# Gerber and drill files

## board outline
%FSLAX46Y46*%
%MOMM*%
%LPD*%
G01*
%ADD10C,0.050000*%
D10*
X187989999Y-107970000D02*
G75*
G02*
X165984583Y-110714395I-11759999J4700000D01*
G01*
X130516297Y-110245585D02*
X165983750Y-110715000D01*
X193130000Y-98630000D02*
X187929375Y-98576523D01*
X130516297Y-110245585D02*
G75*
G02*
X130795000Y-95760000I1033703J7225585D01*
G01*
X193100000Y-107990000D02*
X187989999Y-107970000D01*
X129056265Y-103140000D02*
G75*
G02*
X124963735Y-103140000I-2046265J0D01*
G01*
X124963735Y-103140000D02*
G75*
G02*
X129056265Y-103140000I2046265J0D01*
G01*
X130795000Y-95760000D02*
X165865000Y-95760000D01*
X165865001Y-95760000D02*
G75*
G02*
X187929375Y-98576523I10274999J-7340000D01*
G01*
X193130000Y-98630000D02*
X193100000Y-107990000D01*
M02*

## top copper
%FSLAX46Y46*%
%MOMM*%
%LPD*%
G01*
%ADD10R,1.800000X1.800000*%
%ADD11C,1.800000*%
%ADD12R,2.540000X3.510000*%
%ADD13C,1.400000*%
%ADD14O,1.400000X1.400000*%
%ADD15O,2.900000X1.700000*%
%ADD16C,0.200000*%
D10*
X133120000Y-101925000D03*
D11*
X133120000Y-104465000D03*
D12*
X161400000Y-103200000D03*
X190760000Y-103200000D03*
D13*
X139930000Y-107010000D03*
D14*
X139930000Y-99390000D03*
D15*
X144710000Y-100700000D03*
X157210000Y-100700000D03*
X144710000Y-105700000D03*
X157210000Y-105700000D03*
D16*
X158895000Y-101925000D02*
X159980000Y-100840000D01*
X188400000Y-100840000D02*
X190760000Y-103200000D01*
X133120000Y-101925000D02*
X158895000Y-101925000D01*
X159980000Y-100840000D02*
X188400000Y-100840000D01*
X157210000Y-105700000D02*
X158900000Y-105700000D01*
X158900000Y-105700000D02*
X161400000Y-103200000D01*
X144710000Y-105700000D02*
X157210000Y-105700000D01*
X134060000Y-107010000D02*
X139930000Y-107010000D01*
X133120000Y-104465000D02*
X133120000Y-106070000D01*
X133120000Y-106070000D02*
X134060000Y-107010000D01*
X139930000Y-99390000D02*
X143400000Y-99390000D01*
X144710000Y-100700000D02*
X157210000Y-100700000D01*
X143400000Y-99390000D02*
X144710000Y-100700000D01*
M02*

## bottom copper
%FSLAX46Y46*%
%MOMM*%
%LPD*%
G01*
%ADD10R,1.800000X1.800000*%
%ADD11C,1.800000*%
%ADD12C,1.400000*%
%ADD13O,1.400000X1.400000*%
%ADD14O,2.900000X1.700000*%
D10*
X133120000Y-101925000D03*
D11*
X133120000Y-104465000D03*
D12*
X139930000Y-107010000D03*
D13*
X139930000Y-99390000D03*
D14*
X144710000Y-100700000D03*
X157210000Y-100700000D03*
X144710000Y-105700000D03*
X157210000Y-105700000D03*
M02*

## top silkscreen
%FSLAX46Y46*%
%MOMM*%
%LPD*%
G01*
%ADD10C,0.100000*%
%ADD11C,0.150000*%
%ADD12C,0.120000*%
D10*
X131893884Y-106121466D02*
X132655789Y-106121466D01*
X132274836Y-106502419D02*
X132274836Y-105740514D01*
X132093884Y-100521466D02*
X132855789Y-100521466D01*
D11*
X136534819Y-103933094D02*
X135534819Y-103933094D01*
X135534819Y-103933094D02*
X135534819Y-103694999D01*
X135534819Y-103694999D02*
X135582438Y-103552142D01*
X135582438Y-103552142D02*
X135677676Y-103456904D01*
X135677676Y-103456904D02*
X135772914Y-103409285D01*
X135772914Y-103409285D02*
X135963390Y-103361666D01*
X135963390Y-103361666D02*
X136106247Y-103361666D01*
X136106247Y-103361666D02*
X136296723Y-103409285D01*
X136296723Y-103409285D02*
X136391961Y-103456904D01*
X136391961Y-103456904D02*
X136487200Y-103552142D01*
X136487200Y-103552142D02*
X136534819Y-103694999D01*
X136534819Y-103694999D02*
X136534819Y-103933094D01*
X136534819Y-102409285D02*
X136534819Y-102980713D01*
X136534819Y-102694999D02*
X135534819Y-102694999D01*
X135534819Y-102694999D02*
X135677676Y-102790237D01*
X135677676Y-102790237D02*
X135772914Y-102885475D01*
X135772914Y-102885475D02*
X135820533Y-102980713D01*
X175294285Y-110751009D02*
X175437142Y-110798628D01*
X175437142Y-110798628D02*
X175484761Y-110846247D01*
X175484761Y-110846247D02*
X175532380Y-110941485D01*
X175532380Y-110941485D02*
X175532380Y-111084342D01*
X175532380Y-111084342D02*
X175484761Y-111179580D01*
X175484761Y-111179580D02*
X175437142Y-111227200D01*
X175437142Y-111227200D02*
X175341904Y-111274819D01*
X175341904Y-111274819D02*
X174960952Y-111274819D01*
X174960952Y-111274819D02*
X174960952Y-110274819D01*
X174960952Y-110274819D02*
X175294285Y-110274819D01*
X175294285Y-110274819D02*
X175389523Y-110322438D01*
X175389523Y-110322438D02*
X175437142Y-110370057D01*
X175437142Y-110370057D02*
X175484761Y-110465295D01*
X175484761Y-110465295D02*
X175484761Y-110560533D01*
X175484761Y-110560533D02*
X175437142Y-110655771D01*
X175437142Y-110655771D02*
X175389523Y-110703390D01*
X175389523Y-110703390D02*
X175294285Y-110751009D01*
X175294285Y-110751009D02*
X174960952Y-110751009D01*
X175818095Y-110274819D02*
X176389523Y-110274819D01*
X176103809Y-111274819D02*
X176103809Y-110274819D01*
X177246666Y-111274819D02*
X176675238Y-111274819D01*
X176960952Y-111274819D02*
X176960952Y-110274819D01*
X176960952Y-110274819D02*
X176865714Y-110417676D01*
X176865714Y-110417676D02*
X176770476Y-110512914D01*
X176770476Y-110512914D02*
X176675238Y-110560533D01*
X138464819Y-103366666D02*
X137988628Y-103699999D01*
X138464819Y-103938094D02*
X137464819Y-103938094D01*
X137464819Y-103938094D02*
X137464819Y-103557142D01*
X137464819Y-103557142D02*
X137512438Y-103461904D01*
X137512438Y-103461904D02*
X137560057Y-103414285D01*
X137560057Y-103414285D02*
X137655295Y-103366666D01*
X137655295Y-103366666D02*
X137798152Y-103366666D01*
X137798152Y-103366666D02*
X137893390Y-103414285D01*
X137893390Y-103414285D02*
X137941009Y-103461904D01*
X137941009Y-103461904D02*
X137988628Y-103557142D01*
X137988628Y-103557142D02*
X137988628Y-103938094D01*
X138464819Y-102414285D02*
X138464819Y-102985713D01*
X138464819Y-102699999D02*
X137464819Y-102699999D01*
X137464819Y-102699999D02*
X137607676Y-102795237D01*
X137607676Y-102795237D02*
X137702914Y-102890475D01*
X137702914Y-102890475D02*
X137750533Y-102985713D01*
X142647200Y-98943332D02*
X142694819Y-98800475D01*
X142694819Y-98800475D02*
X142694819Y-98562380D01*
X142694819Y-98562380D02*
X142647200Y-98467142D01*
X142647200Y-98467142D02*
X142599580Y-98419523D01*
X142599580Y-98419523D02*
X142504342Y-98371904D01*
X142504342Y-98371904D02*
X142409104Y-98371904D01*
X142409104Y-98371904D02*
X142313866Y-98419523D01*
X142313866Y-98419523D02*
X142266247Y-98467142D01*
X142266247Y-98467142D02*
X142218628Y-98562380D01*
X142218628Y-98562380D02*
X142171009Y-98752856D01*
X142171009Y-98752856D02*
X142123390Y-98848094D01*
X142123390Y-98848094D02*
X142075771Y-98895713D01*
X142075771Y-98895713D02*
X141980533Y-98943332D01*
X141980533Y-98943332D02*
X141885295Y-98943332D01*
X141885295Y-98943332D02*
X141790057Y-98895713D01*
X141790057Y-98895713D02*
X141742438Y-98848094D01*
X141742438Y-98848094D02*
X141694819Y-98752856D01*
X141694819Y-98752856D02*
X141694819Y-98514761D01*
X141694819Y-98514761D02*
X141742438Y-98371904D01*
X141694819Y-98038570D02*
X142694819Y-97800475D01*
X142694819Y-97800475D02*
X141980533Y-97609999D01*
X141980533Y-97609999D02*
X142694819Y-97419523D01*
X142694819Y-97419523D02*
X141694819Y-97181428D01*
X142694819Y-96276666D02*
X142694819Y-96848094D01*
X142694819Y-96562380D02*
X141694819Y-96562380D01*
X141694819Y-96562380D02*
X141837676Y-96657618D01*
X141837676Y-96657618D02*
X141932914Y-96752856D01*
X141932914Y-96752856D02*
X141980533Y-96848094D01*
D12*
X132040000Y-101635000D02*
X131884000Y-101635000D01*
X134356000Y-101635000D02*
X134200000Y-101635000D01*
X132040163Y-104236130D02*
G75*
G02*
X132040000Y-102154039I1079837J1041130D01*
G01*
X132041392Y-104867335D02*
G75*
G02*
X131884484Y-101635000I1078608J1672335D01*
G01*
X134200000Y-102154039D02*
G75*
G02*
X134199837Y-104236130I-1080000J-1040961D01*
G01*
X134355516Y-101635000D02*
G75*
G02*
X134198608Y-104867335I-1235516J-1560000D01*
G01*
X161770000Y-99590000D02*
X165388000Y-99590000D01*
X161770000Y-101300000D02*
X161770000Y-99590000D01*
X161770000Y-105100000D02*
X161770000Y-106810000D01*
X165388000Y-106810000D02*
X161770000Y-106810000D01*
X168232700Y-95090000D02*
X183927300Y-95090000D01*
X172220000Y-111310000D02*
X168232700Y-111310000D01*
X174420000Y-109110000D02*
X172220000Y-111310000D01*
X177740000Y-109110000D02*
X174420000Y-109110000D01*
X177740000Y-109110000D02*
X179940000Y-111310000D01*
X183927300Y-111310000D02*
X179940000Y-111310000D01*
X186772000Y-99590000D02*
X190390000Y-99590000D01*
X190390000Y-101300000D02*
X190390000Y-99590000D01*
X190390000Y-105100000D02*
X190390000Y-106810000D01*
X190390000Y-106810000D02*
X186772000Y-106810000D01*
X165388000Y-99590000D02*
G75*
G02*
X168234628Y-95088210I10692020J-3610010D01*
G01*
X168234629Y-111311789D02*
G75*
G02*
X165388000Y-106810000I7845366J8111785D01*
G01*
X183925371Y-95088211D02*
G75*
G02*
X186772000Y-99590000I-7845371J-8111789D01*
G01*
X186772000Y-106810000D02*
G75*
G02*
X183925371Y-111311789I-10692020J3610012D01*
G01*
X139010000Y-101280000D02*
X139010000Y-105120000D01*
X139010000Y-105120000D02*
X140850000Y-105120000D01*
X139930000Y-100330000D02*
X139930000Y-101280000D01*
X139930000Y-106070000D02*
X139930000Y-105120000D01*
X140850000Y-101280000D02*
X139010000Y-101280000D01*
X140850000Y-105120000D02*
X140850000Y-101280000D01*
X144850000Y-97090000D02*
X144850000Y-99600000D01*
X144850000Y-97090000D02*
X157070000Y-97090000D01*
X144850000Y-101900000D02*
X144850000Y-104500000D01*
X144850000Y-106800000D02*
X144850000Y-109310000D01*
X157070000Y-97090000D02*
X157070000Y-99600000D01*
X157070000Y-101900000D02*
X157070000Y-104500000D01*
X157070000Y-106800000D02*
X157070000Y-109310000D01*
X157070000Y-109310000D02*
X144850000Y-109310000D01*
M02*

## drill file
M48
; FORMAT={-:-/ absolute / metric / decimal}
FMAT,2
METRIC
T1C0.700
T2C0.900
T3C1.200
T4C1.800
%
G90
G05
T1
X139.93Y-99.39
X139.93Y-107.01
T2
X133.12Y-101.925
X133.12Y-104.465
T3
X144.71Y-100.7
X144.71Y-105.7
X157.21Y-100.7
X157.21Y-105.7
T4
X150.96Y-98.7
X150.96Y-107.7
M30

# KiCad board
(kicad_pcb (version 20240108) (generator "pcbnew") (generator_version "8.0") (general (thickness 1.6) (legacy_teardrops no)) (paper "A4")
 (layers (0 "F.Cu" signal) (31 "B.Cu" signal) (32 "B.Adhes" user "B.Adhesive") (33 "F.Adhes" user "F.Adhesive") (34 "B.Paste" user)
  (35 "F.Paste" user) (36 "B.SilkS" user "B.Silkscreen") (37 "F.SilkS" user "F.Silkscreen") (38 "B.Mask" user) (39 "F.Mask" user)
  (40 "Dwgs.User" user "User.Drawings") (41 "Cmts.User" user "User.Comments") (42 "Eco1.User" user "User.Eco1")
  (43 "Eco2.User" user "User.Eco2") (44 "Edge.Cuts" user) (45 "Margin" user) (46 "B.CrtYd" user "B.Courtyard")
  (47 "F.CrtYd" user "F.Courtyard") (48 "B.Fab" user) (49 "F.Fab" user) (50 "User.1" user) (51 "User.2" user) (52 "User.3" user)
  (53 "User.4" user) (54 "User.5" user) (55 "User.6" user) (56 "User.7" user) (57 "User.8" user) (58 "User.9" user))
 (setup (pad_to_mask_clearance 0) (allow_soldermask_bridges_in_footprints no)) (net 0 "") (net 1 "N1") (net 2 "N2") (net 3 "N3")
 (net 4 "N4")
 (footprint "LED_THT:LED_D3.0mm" (layer "F.Cu") (at 133.12 101.925 -90)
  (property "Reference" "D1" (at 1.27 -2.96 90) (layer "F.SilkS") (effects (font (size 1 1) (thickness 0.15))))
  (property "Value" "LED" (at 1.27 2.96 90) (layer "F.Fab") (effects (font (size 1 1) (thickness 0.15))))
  (fp_line (start -0.29 1.08) (end -0.29 1.236) (stroke (width 0.12) (type solid)) (layer "F.SilkS"))
  (fp_line (start -0.29 -1.236) (end -0.29 -1.08) (stroke (width 0.12) (type solid)) (layer "F.SilkS"))
  (fp_arc (start 2.31113 1.079837) (mid 1.270117 1.5) (end 0.229039 1.08) (stroke (width 0.12) (type solid)) (layer "F.SilkS"))
  (fp_arc (start 2.942335 1.078608) (mid 1.366487 1.987659) (end -0.29 1.235516) (stroke (width 0.12) (type solid)) (layer "F.SilkS"))
  (fp_arc (start 0.229039 -1.08) (mid 1.270117 -1.5) (end 2.31113 -1.079837) (stroke (width 0.12) (type solid)) (layer "F.SilkS"))
  (fp_arc (start -0.29 -1.235516) (mid 1.366487 -1.987659) (end 2.942335 -1.078608) (stroke (width 0.12) (type solid)) (layer "F.SilkS"))
  (pad "1" thru_hole rect (at 0 0 270) (size 1.8 1.8) (drill 0.9) (layers "*.Cu" "*.Mask") (remove_unused_layers no) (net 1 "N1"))
  (pad "2" thru_hole circle (at 2.54 0 270) (size 1.8 1.8) (drill 0.9) (layers "*.Cu" "*.Mask") (remove_unused_layers no) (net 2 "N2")))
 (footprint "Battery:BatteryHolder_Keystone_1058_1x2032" (layer "F.Cu") (at 176.08 103.2)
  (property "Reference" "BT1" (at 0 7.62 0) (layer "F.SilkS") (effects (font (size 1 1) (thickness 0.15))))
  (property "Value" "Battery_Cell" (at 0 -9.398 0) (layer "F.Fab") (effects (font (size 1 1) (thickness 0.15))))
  (fp_line (start -14.31 -3.61) (end -10.692 -3.61) (stroke (width 0.12) (type solid)) (layer "F.SilkS"))
  (fp_line (start -14.31 -1.9) (end -14.31 -3.61) (stroke (width 0.12) (type solid)) (layer "F.SilkS"))
  (fp_line (start -14.31 1.9) (end -14.31 3.61) (stroke (width 0.12) (type solid)) (layer "F.SilkS"))
  (fp_line (start -10.692 3.61) (end -14.31 3.61) (stroke (width 0.12) (type solid)) (layer "F.SilkS"))
  (fp_line (start -7.8473 -8.11) (end 7.8473 -8.11) (stroke (width 0.12) (type solid)) (layer "F.SilkS"))
  (fp_line (start -3.86 8.11) (end -7.8473 8.11) (stroke (width 0.12) (type solid)) (layer "F.SilkS"))
  (fp_line (start -1.66 5.91) (end -3.86 8.11) (stroke (width 0.12) (type solid)) (layer "F.SilkS"))
  (fp_line (start 1.66 5.91) (end -1.66 5.91) (stroke (width 0.12) (type solid)) (layer "F.SilkS"))
  (fp_line (start 1.66 5.91) (end 3.86 8.11) (stroke (width 0.12) (type solid)) (layer "F.SilkS"))
  (fp_line (start 7.8473 8.11) (end 3.86 8.11) (stroke (width 0.12) (type solid)) (layer "F.SilkS"))
  (fp_line (start 10.692 -3.61) (end 14.31 -3.61) (stroke (width 0.12) (type solid)) (layer "F.SilkS"))
  (fp_line (start 14.31 -1.9) (end 14.31 -3.61) (stroke (width 0.12) (type solid)) (layer "F.SilkS"))
  (fp_line (start 14.31 1.9) (end 14.31 3.61) (stroke (width 0.12) (type solid)) (layer "F.SilkS"))
  (fp_line (start 14.31 3.61) (end 10.692 3.61) (stroke (width 0.12) (type solid)) (layer "F.SilkS"))
  (fp_arc (start -10.692 -3.61) (mid -9.538084 -6.031244) (end -7.845371 -8.111789) (stroke (width 0.12) (type solid)) (layer "F.SilkS"))
  (fp_arc (start -7.845371 8.111789) (mid -9.538085 6.031244) (end -10.692 3.61) (stroke (width 0.12) (type solid)) (layer "F.SilkS"))
  (fp_arc (start 7.845371 -8.111789) (mid 9.538085 -6.031244) (end 10.692 -3.61) (stroke (width 0.12) (type solid)) (layer "F.SilkS"))
  (fp_arc (start 10.692 3.61) (mid 9.538084 6.031244) (end 7.845371 8.111789) (stroke (width 0.12) (type solid)) (layer "F.SilkS"))
  (pad "1" smd rect (at -14.68 0) (size 2.54 3.51) (layers "F.Cu" "F.Paste" "F.Mask") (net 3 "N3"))
  (pad "2" smd rect (at 14.68 0) (size 2.54 3.51) (layers "F.Cu" "F.Paste" "F.Mask") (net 1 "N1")))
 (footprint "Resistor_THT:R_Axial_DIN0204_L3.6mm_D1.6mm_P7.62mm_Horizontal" (layer "F.Cu") (at 139.93 107.01 90)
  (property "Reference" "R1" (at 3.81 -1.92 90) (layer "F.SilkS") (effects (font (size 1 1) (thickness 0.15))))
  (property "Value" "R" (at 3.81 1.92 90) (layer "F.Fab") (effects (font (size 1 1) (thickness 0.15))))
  (fp_line (start 5.73 -0.92) (end 1.89 -0.92) (stroke (width 0.12) (type solid)) (layer "F.SilkS"))
  (fp_line (start 1.89 -0.92) (end 1.89 0.92) (stroke (width 0.12) (type solid)) (layer "F.SilkS"))
  (fp_line (start 6.68 0) (end 5.73 0) (stroke (width 0.12) (type solid)) (layer "F.SilkS"))
  (fp_line (start 0.94 0) (end 1.89 0) (stroke (width 0.12) (type solid)) (layer "F.SilkS"))
  (fp_line (start 5.73 0.92) (end 5.73 -0.92) (stroke (width 0.12) (type solid)) (layer "F.SilkS"))
  (fp_line (start 1.89 0.92) (end 5.73 0.92) (stroke (width 0.12) (type solid)) (layer "F.SilkS"))
  (pad "1" thru_hole circle (at 0 0 90) (size 1.4 1.4) (drill 0.7) (layers "*.Cu" "*.Mask") (remove_unused_layers no) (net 2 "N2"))
  (pad "2" thru_hole oval (at 7.62 0 90) (size 1.4 1.4) (drill 0.7) (layers "*.Cu" "*.Mask") (remove_unused_layers no) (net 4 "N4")))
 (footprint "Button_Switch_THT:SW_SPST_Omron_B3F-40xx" (layer "F.Cu") (at 144.71 100.7)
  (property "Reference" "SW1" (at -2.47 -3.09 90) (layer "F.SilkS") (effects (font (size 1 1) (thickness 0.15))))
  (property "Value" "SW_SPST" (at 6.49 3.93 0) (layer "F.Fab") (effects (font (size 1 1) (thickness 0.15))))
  (fp_line (start 0.14 -3.61) (end 0.14 -1.1) (stroke (width 0.12) (type default)) (layer "F.SilkS"))
  (fp_line (start 0.14 -3.61) (end 12.36 -3.61) (stroke (width 0.12) (type default)) (layer "F.SilkS"))
  (fp_line (start 0.14 1.2) (end 0.14 3.8) (stroke (width 0.12) (type default)) (layer "F.SilkS"))
  (fp_line (start 0.14 6.1) (end 0.14 8.61) (stroke (width 0.12) (type default)) (layer "F.SilkS"))
  (fp_line (start 12.36 -3.61) (end 12.36 -1.1) (stroke (width 0.12) (type default)) (layer "F.SilkS"))
  (fp_line (start 12.36 1.2) (end 12.36 3.8) (stroke (width 0.12) (type default)) (layer "F.SilkS"))
  (fp_line (start 12.36 6.1) (end 12.36 8.61) (stroke (width 0.12) (type default)) (layer "F.SilkS"))
  (fp_line (start 12.36 8.61) (end 0.14 8.61) (stroke (width 0.12) (type default)) (layer "F.SilkS"))
  (pad "" np_thru_hole circle (at 6.25 -2) (size 1.8 1.8) (drill 1.8) (layers "F&B.Cu" "*.Mask"))
  (pad "" np_thru_hole circle (at 6.25 7) (size 1.8 1.8) (drill 1.8) (layers "F&B.Cu" "*.Mask"))
  (pad "1" thru_hole oval (at 0 0) (size 2.9 1.7) (drill 1.2) (layers "*.Cu" "*.Mask") (remove_unused_layers no) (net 4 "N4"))
  (pad "1" thru_hole oval (at 12.5 0) (size 2.9 1.7) (drill 1.2) (layers "*.Cu" "*.Mask") (remove_unused_layers no) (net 4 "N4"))
  (pad "2" thru_hole oval (at 0 5) (size 2.9 1.7) (drill 1.2) (layers "*.Cu" "*.Mask") (remove_unused_layers no) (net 3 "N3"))
  (pad "2" thru_hole oval (at 12.5 5) (size 2.9 1.7) (drill 1.2) (layers "*.Cu" "*.Mask") (remove_unused_layers no) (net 3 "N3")))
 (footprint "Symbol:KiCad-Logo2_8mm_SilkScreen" (layer "B.Cu") (at 173.409893 102.476424 180)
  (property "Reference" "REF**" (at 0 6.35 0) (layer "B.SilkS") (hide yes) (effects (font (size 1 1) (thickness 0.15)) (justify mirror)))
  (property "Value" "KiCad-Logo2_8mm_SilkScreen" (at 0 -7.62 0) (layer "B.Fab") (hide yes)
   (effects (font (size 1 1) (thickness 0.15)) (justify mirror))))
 (gr_arc (start 187.989999 107.97) (mid 177.797296 115.837067) (end 165.984583 110.714395) (stroke (width 0.05) (type default))
  (layer "Edge.Cuts"))
 (gr_line (start 130.516297 110.245585) (end 165.98375 110.715) (stroke (width 0.05) (type default)) (layer "Edge.Cuts"))
 (gr_line (start 193.13 98.63) (end 187.929375 98.576523) (stroke (width 0.05) (type default)) (layer "Edge.Cuts"))
 (gr_arc (start 130.516297 110.245585) (mid 124.252199 102.87959) (end 130.795 95.76) (stroke (width 0.05) (type default))
  (layer "Edge.Cuts"))
 (gr_line (start 193.1 107.99) (end 187.989999 107.97) (stroke (width 0.05) (type default)) (layer "Edge.Cuts"))
 (gr_circle (center 127.01 103.14) (end 126.85 101.1) (stroke (width 0.05) (type default)) (fill none) (layer "Edge.Cuts"))
 (gr_line (start 130.795 95.76) (end 165.865 95.76) (stroke (width 0.05) (type default)) (layer "Edge.Cuts"))
 (gr_arc (start 165.865001 95.76) (mid 177.738917 90.57424) (end 187.929375 98.576523) (stroke (width 0.05) (type default))
  (layer "Edge.Cuts"))
 (gr_line (start 193.13 98.63) (end 193.1 107.99) (stroke (width 0.05) (type default)) (layer "Edge.Cuts"))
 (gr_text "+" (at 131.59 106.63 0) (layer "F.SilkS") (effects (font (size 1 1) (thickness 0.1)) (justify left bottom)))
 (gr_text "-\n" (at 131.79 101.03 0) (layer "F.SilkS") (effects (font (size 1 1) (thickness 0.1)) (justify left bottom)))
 (segment (start 158.895 101.925) (end 159.98 100.84) (width 0.2) (layer "F.Cu") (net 1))
 (segment (start 188.4 100.84) (end 190.76 103.2) (width 0.2) (layer "F.Cu") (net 1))
 (segment (start 133.12 101.925) (end 158.895 101.925) (width 0.2) (layer "F.Cu") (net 1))
 (segment (start 159.98 100.84) (end 188.4 100.84) (width 0.2) (layer "F.Cu") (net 1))
 (segment (start 157.21 105.7) (end 158.9 105.7) (width 0.2) (layer "F.Cu") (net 3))
 (segment (start 158.9 105.7) (end 161.4 103.2) (width 0.2) (layer "F.Cu") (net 3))
 (segment (start 144.71 105.7) (end 157.21 105.7) (width 0.2) (layer "F.Cu") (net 3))
 (segment (start 134.06 107.01) (end 139.93 107.01) (width 0.2) (layer "F.Cu") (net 2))
 (segment (start 133.12 104.465) (end 133.12 106.07) (width 0.2) (layer "F.Cu") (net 2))
 (segment (start 133.12 106.07) (end 134.06 107.01) (width 0.2) (layer "F.Cu") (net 2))
 (segment (start 139.93 99.39) (end 143.4 99.39) (width 0.2) (layer "F.Cu") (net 4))
 (segment (start 144.71 100.7) (end 157.21 100.7) (width 0.2) (layer "F.Cu") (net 4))
 (segment (start 143.4 99.39) (end 144.71 100.7) (width 0.2) (layer "F.Cu") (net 4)))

